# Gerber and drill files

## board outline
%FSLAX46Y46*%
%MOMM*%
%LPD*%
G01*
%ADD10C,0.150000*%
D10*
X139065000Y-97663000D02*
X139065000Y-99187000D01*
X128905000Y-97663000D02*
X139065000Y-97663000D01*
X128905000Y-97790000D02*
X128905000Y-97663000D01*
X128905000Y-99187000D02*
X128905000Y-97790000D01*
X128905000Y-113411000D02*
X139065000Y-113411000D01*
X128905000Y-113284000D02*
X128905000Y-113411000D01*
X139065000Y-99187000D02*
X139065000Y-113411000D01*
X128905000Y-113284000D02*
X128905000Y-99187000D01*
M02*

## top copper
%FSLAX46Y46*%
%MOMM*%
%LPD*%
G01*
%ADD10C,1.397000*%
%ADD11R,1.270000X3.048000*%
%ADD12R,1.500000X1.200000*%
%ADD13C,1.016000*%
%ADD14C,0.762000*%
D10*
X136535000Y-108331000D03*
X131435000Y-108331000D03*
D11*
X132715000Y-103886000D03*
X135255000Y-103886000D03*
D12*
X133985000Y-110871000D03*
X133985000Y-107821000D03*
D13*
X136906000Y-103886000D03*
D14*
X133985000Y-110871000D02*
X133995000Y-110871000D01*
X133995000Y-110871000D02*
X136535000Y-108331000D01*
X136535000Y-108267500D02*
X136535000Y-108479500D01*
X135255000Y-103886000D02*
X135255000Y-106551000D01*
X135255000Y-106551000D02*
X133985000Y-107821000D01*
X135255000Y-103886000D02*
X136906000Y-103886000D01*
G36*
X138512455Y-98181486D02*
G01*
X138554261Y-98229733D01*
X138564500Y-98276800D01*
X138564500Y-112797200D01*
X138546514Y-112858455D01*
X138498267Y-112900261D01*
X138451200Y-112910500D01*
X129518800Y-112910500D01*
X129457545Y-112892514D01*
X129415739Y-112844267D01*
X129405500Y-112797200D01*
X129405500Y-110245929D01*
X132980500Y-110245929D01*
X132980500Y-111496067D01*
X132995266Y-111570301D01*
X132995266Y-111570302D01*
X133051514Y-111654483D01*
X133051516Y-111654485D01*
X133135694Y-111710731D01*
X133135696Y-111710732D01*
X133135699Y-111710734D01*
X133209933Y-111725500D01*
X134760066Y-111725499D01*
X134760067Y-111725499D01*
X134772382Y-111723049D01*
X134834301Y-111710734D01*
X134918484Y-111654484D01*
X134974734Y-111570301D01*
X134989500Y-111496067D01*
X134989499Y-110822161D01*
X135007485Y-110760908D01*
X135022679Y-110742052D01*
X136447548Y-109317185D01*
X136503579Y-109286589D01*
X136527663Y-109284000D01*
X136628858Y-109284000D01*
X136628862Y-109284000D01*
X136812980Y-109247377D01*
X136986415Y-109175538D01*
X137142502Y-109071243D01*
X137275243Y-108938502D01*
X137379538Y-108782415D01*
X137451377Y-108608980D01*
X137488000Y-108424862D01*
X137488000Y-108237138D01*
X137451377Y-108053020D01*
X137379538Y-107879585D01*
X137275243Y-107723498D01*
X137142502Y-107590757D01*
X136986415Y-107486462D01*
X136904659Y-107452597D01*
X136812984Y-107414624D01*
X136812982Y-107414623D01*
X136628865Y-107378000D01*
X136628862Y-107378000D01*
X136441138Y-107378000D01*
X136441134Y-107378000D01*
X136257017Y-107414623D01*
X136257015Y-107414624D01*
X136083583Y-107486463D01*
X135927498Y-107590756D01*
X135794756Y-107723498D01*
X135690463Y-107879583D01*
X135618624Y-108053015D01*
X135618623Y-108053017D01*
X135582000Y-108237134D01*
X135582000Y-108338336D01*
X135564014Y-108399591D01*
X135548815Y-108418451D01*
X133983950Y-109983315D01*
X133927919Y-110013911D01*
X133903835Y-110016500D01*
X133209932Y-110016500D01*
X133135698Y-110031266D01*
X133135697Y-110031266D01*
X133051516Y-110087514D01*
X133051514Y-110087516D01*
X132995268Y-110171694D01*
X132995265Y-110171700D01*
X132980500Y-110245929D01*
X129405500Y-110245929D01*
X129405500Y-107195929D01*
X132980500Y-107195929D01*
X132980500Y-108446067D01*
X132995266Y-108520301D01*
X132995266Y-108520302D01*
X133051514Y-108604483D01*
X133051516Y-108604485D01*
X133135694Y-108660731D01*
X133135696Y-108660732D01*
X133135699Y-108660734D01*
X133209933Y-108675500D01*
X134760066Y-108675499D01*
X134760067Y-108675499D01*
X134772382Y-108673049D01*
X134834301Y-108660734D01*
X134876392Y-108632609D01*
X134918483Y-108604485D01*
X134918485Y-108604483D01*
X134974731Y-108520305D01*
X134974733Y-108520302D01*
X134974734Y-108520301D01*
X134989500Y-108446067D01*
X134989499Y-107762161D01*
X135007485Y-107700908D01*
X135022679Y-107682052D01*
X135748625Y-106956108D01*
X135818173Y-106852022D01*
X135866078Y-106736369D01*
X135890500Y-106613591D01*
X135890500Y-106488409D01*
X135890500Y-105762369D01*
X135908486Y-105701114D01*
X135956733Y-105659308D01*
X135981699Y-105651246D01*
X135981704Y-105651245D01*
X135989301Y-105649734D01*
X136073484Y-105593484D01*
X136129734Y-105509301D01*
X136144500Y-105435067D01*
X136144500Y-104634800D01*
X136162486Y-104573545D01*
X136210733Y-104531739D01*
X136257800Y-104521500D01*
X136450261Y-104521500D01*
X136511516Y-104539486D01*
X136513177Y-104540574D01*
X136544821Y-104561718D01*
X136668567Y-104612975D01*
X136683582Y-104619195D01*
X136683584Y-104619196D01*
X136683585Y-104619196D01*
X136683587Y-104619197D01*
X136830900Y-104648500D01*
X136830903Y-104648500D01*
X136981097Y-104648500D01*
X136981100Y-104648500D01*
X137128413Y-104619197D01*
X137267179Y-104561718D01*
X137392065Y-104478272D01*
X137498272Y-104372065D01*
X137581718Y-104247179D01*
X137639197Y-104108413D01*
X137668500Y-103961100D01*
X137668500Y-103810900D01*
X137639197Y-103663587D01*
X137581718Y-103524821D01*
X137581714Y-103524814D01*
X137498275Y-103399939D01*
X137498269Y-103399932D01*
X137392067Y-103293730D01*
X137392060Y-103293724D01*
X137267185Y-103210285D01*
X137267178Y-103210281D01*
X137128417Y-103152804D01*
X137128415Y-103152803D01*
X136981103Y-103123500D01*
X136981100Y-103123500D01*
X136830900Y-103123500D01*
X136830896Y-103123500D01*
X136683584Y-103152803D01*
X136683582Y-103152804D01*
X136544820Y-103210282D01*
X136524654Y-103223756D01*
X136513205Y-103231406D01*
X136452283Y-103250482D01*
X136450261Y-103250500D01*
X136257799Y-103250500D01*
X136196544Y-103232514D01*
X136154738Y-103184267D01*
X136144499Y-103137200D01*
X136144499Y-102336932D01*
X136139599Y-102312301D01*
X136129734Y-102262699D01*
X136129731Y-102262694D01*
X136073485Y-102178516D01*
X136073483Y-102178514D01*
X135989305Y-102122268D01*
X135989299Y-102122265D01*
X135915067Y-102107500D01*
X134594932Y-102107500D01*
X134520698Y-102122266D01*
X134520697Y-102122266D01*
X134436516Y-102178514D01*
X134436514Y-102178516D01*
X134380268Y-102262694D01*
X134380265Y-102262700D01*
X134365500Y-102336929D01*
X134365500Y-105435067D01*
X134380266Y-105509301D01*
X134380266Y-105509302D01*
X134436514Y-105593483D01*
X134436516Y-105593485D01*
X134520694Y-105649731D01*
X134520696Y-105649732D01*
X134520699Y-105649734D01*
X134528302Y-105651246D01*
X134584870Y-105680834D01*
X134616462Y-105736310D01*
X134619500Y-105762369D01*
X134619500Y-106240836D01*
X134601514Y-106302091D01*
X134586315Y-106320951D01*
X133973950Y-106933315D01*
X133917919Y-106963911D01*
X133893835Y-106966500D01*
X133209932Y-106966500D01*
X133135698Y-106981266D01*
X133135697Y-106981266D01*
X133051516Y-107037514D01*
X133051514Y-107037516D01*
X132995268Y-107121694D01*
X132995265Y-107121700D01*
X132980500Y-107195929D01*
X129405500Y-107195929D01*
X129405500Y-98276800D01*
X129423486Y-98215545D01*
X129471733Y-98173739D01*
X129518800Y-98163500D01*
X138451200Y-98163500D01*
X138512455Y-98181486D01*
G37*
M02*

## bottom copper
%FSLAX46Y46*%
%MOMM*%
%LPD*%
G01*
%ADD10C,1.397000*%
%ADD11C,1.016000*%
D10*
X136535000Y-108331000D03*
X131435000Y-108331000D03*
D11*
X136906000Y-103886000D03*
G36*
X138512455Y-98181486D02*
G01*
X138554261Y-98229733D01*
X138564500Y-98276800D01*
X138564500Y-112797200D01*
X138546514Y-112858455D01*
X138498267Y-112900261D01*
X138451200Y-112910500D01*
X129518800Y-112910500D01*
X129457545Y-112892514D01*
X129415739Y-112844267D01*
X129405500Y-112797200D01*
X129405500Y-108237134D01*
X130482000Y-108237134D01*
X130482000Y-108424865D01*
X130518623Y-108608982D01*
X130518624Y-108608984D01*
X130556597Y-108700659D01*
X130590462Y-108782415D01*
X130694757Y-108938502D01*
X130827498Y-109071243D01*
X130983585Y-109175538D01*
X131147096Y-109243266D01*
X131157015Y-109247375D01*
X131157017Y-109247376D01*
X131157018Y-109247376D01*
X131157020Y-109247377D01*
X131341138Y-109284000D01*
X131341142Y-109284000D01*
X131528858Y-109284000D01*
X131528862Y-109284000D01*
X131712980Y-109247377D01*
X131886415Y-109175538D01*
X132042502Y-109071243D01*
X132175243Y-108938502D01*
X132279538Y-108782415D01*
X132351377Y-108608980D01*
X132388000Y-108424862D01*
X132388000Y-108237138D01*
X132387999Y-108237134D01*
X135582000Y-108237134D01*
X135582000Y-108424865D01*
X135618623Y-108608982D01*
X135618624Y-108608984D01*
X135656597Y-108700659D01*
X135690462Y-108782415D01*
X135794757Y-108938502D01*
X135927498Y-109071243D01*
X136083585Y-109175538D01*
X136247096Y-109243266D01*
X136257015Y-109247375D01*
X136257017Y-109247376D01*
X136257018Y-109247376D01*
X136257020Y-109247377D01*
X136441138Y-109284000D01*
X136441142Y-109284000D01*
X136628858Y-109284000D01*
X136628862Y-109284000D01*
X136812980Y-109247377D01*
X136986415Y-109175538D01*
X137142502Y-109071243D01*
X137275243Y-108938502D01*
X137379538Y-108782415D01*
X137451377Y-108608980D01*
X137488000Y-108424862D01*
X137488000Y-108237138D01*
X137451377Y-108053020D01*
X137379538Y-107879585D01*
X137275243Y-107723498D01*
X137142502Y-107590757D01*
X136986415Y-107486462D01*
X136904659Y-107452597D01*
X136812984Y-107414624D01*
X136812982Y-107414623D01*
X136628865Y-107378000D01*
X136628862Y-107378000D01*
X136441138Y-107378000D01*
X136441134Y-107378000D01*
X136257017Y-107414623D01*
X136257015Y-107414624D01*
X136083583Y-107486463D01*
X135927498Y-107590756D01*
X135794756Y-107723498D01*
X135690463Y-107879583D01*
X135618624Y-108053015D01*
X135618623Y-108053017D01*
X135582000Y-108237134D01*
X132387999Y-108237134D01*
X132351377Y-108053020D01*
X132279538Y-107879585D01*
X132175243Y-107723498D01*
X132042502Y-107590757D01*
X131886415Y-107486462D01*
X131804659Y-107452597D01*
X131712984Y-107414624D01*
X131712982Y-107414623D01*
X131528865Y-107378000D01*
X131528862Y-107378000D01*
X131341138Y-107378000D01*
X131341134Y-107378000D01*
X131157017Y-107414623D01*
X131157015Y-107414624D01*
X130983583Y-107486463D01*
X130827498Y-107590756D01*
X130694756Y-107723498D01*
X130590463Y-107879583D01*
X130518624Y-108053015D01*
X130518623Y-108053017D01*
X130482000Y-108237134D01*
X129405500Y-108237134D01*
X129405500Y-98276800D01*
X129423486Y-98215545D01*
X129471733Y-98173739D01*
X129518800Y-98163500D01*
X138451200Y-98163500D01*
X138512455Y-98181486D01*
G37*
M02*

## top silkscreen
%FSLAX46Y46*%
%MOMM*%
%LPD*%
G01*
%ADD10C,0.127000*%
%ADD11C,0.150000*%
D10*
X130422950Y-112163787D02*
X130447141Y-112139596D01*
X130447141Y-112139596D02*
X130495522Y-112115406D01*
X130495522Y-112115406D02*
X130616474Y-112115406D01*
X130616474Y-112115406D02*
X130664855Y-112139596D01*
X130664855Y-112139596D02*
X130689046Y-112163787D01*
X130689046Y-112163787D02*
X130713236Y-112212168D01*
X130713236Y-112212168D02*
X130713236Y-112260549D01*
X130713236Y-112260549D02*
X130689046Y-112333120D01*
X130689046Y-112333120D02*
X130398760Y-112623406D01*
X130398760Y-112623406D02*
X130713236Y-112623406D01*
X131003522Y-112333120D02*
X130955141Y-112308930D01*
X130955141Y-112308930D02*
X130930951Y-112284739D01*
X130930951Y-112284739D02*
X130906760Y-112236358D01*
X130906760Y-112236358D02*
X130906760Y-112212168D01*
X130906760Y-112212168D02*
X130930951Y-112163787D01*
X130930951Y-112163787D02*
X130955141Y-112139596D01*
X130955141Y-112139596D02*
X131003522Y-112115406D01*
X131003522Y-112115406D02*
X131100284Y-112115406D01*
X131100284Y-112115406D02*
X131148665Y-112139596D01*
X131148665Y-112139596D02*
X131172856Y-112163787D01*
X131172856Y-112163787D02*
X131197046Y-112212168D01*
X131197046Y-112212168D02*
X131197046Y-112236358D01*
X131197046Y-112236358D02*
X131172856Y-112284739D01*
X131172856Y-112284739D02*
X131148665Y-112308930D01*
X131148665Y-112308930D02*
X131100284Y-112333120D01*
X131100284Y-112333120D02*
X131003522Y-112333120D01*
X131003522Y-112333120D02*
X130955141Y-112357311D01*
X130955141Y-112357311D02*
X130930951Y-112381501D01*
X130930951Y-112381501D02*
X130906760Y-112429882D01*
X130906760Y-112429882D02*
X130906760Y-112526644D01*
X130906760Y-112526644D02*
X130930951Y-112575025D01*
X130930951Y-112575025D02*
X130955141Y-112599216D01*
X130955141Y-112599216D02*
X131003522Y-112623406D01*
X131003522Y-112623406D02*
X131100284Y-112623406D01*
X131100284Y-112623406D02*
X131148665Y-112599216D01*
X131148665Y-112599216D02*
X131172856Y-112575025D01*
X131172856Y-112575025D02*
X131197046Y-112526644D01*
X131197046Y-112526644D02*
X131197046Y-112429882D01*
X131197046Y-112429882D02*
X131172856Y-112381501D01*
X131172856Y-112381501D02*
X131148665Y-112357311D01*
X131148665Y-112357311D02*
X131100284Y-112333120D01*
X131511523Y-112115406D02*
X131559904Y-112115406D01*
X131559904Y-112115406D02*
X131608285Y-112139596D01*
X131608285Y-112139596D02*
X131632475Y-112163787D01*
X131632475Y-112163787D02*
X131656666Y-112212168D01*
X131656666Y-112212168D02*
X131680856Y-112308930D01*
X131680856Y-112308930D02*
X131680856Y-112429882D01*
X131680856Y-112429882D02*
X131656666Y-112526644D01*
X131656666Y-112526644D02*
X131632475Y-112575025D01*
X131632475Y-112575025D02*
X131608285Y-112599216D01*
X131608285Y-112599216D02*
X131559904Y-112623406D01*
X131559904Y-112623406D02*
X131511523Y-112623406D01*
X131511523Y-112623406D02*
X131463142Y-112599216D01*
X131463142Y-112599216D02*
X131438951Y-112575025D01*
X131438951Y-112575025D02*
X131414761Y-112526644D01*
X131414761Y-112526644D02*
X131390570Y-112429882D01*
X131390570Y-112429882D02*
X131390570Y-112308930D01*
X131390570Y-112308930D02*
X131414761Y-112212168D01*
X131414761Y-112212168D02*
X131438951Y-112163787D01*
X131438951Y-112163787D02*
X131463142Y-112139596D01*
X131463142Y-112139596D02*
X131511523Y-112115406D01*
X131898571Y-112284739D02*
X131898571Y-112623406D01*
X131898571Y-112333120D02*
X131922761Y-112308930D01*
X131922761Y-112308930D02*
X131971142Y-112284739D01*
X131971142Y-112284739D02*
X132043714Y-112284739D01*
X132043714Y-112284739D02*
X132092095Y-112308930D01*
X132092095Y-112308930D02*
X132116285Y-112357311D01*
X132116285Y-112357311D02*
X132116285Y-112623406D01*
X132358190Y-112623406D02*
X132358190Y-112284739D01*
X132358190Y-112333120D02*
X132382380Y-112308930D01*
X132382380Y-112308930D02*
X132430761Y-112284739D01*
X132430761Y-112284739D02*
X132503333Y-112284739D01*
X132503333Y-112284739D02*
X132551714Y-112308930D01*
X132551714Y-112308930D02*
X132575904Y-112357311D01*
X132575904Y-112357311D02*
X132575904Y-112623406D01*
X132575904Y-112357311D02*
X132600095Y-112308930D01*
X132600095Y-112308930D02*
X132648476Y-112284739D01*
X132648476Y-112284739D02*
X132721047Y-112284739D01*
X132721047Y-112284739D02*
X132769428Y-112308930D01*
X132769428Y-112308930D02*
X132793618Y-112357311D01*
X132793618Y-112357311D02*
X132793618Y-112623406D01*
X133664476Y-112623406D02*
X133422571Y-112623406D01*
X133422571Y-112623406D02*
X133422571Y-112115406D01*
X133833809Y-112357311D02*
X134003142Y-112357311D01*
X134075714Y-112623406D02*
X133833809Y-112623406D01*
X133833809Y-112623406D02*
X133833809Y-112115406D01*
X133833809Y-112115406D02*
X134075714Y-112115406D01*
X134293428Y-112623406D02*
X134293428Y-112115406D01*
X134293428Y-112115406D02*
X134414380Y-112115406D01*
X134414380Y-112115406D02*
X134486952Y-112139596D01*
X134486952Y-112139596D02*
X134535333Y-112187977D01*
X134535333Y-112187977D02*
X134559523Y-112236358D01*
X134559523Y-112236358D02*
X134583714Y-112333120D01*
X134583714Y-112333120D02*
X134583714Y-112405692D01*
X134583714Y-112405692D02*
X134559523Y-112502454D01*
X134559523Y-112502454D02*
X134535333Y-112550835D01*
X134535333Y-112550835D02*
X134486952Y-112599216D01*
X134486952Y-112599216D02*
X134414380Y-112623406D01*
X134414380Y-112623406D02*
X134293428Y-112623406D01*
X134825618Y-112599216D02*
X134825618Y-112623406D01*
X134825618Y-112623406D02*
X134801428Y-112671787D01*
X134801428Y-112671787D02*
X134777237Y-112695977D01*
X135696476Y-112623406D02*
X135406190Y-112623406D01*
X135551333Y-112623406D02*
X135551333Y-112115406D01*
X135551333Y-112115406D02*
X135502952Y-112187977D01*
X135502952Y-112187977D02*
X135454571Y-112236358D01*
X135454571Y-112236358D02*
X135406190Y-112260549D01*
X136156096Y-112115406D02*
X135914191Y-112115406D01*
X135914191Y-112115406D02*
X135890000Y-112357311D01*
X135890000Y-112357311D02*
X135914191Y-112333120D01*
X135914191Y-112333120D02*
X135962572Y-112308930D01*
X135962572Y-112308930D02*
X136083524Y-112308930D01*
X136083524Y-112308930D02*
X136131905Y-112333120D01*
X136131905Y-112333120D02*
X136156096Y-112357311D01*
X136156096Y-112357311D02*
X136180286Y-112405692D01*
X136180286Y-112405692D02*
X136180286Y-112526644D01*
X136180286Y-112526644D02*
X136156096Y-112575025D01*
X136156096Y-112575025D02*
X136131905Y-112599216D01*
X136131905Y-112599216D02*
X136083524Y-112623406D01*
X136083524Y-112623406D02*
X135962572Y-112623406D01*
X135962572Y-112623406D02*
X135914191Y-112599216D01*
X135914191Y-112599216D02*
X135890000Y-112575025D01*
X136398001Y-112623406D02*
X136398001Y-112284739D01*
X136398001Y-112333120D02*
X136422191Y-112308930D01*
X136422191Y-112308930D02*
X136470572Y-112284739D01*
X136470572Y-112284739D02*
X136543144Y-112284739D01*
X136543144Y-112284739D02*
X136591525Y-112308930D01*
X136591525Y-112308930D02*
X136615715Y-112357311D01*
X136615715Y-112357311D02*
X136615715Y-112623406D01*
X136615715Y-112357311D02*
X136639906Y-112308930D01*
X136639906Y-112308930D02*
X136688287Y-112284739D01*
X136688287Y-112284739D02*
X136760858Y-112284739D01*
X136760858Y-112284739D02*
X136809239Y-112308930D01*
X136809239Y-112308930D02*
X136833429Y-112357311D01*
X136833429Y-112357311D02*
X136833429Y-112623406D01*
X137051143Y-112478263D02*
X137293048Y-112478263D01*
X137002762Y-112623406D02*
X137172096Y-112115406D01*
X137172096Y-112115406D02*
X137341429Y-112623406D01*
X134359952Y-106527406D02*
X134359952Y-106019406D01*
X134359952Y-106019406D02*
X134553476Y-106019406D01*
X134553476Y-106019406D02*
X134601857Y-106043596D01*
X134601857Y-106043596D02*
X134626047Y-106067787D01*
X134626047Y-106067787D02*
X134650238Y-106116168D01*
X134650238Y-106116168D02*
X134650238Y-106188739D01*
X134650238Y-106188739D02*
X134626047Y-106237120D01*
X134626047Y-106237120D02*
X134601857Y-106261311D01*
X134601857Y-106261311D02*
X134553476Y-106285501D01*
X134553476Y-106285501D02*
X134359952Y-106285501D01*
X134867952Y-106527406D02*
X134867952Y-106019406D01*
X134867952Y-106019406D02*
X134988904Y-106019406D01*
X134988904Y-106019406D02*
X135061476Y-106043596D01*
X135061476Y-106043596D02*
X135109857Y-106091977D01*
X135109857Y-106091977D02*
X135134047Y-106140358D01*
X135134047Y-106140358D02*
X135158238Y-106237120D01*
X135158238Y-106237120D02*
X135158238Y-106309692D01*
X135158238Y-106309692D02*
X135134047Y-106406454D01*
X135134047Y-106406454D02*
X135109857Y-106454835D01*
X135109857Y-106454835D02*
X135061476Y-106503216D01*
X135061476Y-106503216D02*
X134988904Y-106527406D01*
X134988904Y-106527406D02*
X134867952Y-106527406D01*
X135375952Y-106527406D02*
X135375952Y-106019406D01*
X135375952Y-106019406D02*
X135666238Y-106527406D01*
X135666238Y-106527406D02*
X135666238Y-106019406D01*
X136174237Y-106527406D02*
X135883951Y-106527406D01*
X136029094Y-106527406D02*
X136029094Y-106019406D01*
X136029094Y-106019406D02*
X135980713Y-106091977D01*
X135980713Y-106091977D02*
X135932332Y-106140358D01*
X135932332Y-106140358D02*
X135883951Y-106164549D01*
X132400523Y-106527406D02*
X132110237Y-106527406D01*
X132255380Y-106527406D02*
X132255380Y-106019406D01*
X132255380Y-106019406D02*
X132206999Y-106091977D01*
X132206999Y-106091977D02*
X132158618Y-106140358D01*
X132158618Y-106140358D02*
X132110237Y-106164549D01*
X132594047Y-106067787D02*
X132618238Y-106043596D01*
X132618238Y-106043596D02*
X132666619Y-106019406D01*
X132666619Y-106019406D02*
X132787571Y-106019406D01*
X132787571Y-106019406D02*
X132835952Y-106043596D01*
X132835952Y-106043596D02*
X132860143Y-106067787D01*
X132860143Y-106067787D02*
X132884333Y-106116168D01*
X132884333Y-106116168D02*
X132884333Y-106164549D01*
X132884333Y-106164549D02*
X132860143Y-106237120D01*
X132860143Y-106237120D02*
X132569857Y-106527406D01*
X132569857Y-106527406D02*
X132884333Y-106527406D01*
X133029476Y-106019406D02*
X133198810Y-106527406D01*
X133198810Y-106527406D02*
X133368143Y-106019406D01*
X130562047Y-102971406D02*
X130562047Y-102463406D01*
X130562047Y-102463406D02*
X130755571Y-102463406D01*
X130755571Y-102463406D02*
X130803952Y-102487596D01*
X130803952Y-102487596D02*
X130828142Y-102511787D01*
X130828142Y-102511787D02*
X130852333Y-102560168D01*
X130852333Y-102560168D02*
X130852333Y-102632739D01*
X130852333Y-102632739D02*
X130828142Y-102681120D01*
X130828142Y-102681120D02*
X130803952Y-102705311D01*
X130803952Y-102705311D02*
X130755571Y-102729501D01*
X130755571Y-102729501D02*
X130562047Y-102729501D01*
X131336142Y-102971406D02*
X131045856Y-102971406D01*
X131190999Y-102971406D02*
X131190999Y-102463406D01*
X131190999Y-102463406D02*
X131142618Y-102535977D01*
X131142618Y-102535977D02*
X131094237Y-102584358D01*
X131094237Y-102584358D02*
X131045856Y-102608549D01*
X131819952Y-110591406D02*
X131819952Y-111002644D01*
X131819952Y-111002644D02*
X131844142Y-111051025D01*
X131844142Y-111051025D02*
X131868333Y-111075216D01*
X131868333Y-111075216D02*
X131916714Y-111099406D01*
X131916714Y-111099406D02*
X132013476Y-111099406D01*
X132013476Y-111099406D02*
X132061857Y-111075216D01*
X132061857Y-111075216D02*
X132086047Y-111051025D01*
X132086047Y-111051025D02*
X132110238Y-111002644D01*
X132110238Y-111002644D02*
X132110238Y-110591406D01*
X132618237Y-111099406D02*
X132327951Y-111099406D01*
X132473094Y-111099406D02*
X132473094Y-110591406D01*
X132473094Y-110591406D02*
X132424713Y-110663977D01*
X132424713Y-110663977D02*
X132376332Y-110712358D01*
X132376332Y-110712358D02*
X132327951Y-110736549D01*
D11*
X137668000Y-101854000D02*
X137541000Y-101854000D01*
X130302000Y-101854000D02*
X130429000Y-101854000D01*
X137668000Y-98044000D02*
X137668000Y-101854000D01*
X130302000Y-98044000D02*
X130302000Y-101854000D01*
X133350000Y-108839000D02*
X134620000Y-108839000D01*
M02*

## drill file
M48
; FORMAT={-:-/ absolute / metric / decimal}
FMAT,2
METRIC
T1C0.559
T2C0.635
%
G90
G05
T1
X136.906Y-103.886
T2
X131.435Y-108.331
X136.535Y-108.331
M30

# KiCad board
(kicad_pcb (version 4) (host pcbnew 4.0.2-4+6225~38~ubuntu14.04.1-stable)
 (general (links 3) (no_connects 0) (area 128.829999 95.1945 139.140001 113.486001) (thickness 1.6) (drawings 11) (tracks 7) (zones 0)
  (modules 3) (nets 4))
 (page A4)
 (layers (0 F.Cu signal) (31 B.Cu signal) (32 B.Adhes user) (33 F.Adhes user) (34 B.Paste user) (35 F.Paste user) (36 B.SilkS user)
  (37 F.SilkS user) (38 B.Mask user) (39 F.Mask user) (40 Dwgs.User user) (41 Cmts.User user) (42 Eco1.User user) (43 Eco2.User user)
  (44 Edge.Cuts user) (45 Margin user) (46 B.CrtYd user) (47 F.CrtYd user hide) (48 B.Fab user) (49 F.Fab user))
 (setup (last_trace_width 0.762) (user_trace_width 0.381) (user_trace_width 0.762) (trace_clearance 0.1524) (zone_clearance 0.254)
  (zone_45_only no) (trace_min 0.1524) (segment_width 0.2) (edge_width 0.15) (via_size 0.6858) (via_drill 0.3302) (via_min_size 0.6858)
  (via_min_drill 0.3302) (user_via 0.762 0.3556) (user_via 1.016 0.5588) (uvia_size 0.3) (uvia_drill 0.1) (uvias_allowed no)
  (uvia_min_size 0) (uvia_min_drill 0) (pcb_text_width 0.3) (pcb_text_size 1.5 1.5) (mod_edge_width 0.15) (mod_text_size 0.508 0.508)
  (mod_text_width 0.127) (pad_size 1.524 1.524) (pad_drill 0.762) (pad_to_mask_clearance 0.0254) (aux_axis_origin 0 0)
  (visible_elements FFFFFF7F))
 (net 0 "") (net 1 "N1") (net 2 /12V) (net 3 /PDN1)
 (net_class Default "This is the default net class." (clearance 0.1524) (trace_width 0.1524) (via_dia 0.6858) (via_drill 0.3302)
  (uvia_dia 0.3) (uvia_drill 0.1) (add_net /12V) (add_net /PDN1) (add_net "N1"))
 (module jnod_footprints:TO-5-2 (layer B.Cu) (at 133.985 108.331 180)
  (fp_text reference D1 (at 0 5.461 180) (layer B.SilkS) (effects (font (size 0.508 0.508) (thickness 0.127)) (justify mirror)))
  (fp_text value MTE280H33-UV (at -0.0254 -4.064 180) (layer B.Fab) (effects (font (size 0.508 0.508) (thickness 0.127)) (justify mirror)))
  (pad 1 thru_hole circle (at -2.55 0 180) (size 1.397 1.397) (drill 0.635) (layers *.Cu *.Mask B.SilkS) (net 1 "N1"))
  (pad 2 thru_hole circle (at 2.55 0 180) (size 1.397 1.397) (drill 0.635) (layers *.Cu *.Mask B.SilkS) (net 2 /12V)))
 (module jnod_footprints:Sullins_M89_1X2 (layer F.Cu) (at 132.715 103.886)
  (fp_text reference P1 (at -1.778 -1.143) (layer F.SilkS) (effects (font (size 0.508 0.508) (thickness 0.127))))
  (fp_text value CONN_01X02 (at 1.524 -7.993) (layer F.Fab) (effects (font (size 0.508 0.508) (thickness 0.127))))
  (fp_line (start 4.953 -2.032) (end 4.826 -2.032) (layer F.SilkS) (width 0.15))
  (fp_line (start -2.413 -2.032) (end -2.286 -2.032) (layer F.SilkS) (width 0.15))
  (fp_line (start 4.953 -5.842) (end 4.953 -2.032) (layer F.SilkS) (width 0.15))
  (fp_line (start -2.413 -5.842) (end -2.413 -2.032) (layer F.SilkS) (width 0.15))
  (pad 1 smd rect (at 0 0) (size 1.27 3.048) (layers F.Cu F.Paste F.Mask) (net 2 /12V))
  (pad 2 smd rect (at 2.54 0) (size 1.27 3.048) (layers F.Cu F.Paste F.Mask) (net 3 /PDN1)))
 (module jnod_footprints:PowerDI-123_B (layer F.Cu) (at 133.985 110.871 90)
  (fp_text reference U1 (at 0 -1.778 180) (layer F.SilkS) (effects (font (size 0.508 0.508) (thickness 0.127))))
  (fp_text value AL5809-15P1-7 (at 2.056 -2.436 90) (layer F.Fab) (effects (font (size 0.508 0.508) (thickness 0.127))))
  (fp_line (start 2.032 -0.635) (end 2.032 0.635) (layer F.SilkS) (width 0.15))
  (pad 1 smd rect (at 0 0 90) (size 1.2 1.5) (layers F.Cu F.Paste F.Mask) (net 1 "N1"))
  (pad 2 smd rect (at 3.05 0 90) (size 1.2 1.5) (layers F.Cu F.Paste F.Mask) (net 3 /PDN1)))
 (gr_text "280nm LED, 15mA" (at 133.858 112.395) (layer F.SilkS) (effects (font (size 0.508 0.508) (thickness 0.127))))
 (gr_line (start 139.065 97.663) (end 139.065 99.187) (angle 90) (layer Edge.Cuts) (width 0.15))
 (gr_line (start 128.905 97.663) (end 139.065 97.663) (angle 90) (layer Edge.Cuts) (width 0.15))
 (gr_line (start 128.905 97.79) (end 128.905 97.663) (angle 90) (layer Edge.Cuts) (width 0.15))
 (gr_line (start 128.905 99.187) (end 128.905 97.79) (angle 90) (layer Edge.Cuts) (width 0.15))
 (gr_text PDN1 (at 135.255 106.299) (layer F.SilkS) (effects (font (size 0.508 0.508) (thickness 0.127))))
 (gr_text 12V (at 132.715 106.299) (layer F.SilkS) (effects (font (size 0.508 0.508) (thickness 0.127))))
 (gr_line (start 128.905 113.411) (end 139.065 113.411) (angle 90) (layer Edge.Cuts) (width 0.15))
 (gr_line (start 128.905 113.284) (end 128.905 113.411) (angle 90) (layer Edge.Cuts) (width 0.15))
 (gr_line (start 139.065 99.187) (end 139.065 113.411) (angle 90) (layer Edge.Cuts) (width 0.15))
 (gr_line (start 128.905 113.284) (end 128.905 99.187) (angle 90) (layer Edge.Cuts) (width 0.15))
 (segment (start 133.985 110.871) (end 133.995 110.871) (width 0.762) (layer F.Cu) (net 1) (status C00000))
 (segment (start 133.995 110.871) (end 136.535 108.331) (width 0.762) (layer F.Cu) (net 1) (status C00000))
 (segment (start 136.535 108.2675) (end 136.535 108.4795) (width 0.762) (layer F.Cu) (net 1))
 (segment (start 135.255 103.886) (end 135.255 106.551) (width 0.762) (layer F.Cu) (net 3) (status 400000))
 (segment (start 135.255 106.551) (end 133.985 107.821) (width 0.762) (layer F.Cu) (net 3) (status 800000))
 (segment (start 135.255 103.886) (end 136.906 103.886) (width 0.762) (layer F.Cu) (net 3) (status 400000))
 (via (at 136.906 103.886) (size 1.016) (drill 0.5588) (layers F.Cu B.Cu) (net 3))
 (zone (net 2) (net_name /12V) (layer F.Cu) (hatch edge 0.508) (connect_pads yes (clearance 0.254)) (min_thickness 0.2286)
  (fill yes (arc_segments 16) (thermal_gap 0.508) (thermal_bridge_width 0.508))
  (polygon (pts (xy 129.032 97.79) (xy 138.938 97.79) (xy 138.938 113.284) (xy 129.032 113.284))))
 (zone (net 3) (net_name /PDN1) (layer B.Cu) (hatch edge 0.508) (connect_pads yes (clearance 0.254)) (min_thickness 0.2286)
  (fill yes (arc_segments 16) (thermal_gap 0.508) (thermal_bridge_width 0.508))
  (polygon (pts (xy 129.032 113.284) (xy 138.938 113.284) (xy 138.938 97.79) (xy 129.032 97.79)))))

